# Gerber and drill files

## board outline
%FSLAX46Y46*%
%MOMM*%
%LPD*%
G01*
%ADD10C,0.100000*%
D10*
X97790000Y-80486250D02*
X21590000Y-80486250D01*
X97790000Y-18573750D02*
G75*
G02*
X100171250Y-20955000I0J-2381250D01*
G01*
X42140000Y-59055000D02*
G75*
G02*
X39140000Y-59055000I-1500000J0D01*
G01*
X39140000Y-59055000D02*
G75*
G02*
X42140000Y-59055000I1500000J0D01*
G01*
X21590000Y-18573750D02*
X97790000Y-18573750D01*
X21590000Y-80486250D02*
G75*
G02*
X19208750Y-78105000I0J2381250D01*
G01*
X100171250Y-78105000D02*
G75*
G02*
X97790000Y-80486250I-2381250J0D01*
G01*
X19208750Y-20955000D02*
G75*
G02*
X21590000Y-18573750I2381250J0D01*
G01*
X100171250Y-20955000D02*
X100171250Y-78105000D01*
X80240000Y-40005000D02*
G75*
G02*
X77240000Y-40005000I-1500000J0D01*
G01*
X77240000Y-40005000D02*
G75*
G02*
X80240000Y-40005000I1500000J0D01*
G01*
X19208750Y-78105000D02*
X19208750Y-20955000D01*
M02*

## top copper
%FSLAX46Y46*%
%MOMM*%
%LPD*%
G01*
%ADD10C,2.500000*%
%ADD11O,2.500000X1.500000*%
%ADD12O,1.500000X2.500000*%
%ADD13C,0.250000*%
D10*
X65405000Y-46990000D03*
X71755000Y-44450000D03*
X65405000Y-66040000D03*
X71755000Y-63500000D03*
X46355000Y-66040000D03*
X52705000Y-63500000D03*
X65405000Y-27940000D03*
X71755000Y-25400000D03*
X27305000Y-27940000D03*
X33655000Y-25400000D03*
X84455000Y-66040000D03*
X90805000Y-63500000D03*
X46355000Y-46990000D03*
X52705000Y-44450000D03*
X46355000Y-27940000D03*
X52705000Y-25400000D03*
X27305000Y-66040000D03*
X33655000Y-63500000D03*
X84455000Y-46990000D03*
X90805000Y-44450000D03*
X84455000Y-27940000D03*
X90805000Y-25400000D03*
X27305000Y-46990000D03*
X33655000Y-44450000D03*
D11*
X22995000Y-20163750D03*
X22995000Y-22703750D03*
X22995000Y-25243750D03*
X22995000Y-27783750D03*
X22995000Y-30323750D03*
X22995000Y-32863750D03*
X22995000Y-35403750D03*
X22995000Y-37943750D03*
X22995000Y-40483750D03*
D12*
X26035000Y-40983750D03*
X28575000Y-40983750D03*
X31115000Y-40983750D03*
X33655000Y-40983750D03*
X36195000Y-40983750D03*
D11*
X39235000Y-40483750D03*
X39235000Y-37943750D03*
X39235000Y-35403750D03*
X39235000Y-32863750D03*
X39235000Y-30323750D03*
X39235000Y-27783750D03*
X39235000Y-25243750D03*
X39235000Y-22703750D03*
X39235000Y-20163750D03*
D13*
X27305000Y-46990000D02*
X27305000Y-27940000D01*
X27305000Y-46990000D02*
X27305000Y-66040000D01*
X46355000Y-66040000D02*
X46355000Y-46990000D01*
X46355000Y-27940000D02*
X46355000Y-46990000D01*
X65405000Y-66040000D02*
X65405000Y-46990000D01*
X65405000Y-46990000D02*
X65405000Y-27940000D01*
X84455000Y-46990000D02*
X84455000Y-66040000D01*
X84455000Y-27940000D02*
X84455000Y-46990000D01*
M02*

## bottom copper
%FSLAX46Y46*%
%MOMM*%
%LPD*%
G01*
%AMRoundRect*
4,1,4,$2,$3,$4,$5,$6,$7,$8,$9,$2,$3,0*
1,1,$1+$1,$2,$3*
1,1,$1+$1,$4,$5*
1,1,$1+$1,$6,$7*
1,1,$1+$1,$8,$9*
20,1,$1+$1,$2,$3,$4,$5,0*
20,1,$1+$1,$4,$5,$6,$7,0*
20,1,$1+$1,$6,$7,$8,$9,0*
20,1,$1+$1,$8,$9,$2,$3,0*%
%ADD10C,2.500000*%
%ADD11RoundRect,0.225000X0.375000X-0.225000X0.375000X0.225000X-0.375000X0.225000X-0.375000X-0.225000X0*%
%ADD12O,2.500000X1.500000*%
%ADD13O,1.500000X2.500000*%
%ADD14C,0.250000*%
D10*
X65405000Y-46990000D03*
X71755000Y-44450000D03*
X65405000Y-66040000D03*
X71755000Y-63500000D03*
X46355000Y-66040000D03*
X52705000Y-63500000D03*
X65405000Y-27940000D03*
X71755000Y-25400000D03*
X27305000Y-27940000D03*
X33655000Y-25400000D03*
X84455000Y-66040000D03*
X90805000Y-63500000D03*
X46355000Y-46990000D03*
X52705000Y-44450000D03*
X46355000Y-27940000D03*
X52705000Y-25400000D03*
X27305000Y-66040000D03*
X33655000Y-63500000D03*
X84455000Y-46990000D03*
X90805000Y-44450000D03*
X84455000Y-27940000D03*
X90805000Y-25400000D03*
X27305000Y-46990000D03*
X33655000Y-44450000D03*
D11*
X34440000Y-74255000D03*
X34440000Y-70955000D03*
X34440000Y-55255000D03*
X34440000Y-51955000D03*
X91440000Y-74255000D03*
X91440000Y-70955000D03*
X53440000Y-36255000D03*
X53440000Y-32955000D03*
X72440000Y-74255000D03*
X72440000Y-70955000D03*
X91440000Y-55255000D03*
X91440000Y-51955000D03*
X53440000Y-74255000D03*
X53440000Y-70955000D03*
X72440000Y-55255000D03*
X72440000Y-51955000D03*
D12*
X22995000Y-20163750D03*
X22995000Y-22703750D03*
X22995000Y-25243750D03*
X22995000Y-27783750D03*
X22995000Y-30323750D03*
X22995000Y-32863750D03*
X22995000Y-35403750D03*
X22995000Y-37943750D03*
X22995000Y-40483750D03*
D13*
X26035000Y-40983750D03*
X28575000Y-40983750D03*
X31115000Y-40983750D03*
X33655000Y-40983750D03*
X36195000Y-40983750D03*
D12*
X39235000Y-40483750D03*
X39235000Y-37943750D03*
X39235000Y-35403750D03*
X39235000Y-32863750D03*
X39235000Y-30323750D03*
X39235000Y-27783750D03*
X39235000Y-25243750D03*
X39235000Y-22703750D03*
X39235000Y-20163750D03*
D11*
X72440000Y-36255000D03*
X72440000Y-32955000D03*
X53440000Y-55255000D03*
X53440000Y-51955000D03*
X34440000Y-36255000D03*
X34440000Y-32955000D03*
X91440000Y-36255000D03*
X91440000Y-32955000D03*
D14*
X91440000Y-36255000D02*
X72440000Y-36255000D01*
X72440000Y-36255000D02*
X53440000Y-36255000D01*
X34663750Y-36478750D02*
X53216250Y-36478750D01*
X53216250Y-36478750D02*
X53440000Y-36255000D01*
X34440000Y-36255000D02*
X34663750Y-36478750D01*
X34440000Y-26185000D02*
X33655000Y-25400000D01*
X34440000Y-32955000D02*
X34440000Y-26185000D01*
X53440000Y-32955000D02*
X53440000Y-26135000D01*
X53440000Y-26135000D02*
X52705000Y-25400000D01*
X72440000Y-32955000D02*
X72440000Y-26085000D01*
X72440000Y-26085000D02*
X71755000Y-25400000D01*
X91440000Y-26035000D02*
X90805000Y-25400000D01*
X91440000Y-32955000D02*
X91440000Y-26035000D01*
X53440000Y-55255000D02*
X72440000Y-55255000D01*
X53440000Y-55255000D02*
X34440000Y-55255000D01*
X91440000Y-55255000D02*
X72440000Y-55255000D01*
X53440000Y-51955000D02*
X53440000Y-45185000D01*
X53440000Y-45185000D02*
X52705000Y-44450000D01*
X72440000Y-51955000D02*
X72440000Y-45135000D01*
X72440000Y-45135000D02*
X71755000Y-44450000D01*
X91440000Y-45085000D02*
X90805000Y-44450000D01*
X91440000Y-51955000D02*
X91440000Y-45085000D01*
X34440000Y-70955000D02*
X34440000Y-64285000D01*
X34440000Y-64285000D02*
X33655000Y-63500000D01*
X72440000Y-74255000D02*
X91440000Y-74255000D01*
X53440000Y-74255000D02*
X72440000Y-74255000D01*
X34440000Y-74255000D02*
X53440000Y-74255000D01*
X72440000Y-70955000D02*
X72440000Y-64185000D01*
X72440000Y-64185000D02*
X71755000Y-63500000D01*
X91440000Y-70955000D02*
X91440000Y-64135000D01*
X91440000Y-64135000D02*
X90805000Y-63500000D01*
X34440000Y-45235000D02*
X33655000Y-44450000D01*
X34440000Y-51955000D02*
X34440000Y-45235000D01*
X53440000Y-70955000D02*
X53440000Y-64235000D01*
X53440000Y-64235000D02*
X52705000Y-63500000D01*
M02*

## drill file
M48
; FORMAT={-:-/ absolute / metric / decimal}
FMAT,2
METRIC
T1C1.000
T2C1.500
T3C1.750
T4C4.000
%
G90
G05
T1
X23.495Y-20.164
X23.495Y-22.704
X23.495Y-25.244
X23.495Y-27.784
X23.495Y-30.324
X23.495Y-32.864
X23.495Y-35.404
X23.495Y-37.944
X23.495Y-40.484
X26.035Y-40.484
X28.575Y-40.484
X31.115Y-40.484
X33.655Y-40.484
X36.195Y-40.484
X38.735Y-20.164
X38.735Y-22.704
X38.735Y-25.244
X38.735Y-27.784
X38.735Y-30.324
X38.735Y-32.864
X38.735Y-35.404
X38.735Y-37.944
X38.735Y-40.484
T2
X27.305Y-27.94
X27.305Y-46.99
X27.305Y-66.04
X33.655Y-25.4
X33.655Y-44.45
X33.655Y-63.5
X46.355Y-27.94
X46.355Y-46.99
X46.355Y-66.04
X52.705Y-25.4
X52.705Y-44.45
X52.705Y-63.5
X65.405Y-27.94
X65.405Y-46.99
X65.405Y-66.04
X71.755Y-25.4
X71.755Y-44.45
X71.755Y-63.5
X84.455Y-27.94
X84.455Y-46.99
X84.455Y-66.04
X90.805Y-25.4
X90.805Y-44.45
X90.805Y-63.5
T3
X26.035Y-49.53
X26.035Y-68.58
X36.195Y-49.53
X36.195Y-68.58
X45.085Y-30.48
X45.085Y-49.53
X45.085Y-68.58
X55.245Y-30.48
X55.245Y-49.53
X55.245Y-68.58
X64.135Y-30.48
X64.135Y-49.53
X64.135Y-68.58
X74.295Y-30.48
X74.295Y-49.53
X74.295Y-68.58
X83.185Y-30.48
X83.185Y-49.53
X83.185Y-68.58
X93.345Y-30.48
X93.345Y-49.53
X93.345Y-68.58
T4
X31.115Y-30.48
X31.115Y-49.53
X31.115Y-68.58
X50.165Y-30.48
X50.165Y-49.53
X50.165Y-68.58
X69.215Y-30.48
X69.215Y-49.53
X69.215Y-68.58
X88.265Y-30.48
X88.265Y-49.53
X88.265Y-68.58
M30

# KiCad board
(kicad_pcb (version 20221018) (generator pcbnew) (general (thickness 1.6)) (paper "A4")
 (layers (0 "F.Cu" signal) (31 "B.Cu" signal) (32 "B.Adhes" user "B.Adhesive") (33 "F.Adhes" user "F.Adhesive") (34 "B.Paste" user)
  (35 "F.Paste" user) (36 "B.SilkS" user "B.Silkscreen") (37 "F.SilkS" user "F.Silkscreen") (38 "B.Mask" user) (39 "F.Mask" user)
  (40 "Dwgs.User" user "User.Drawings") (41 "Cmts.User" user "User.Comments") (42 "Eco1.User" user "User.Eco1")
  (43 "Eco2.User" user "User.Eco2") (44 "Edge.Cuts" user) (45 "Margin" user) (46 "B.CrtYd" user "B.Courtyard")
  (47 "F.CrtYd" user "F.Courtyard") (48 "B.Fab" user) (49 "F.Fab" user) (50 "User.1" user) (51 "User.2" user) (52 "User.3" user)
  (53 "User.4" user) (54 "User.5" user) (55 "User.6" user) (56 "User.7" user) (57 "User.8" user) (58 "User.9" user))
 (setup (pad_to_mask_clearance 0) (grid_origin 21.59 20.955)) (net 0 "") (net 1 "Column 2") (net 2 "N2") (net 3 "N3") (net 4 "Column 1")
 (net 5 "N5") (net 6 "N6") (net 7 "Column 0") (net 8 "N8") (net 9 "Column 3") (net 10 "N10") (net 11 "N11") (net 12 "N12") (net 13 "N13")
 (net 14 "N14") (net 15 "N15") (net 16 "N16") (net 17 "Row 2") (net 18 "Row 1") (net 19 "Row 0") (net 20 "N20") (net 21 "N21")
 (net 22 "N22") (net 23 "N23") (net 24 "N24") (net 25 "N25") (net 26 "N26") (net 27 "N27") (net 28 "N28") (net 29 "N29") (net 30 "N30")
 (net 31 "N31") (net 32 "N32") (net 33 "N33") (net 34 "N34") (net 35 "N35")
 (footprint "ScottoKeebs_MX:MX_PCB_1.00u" (layer "F.Cu") (at 69.215 49.53)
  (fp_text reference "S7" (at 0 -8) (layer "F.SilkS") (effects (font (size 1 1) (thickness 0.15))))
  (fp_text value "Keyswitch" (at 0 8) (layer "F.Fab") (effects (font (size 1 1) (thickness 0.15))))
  (pad "" np_thru_hole circle (at -5.08 0) (size 1.75 1.75) (drill 1.75) (layers "*.Cu" "*.Mask"))
  (pad "" np_thru_hole circle (at 0 0) (size 4 4) (drill 4) (layers "*.Cu" "*.Mask"))
  (pad "" np_thru_hole circle (at 5.08 0) (size 1.75 1.75) (drill 1.75) (layers "*.Cu" "*.Mask"))
  (pad "1" thru_hole circle (at -3.81 -2.54) (size 2.5 2.5) (drill 1.5) (layers "*.Cu" "*.Mask") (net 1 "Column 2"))
  (pad "2" thru_hole circle (at 2.54 -5.08) (size 2.5 2.5) (drill 1.5) (layers "*.Cu" "*.Mask") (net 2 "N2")))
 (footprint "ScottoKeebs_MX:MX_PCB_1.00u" (layer "F.Cu") (at 69.215 68.58)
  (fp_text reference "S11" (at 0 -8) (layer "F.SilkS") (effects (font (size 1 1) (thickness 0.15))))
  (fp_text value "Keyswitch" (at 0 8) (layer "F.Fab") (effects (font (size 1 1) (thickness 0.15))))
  (pad "" np_thru_hole circle (at -5.08 0) (size 1.75 1.75) (drill 1.75) (layers "*.Cu" "*.Mask"))
  (pad "" np_thru_hole circle (at 0 0) (size 4 4) (drill 4) (layers "*.Cu" "*.Mask"))
  (pad "" np_thru_hole circle (at 5.08 0) (size 1.75 1.75) (drill 1.75) (layers "*.Cu" "*.Mask"))
  (pad "1" thru_hole circle (at -3.81 -2.54) (size 2.5 2.5) (drill 1.5) (layers "*.Cu" "*.Mask") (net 1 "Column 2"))
  (pad "2" thru_hole circle (at 2.54 -5.08) (size 2.5 2.5) (drill 1.5) (layers "*.Cu" "*.Mask") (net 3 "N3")))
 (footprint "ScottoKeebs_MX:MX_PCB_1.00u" (layer "F.Cu") (at 50.165 68.58)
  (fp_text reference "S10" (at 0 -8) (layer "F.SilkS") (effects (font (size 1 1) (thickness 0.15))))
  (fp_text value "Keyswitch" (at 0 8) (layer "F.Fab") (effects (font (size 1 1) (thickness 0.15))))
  (pad "" np_thru_hole circle (at -5.08 0) (size 1.75 1.75) (drill 1.75) (layers "*.Cu" "*.Mask"))
  (pad "" np_thru_hole circle (at 0 0) (size 4 4) (drill 4) (layers "*.Cu" "*.Mask"))
  (pad "" np_thru_hole circle (at 5.08 0) (size 1.75 1.75) (drill 1.75) (layers "*.Cu" "*.Mask"))
  (pad "1" thru_hole circle (at -3.81 -2.54) (size 2.5 2.5) (drill 1.5) (layers "*.Cu" "*.Mask") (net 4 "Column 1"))
  (pad "2" thru_hole circle (at 2.54 -5.08) (size 2.5 2.5) (drill 1.5) (layers "*.Cu" "*.Mask") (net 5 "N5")))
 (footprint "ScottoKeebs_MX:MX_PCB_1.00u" (layer "F.Cu") (at 69.215 30.48)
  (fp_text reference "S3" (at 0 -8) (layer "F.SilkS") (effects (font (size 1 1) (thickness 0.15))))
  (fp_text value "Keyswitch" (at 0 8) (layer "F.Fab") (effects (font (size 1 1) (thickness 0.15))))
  (pad "" np_thru_hole circle (at -5.08 0) (size 1.75 1.75) (drill 1.75) (layers "*.Cu" "*.Mask"))
  (pad "" np_thru_hole circle (at 0 0) (size 4 4) (drill 4) (layers "*.Cu" "*.Mask"))
  (pad "" np_thru_hole circle (at 5.08 0) (size 1.75 1.75) (drill 1.75) (layers "*.Cu" "*.Mask"))
  (pad "1" thru_hole circle (at -3.81 -2.54) (size 2.5 2.5) (drill 1.5) (layers "*.Cu" "*.Mask") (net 1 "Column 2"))
  (pad "2" thru_hole circle (at 2.54 -5.08) (size 2.5 2.5) (drill 1.5) (layers "*.Cu" "*.Mask") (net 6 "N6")))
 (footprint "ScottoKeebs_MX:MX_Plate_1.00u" (layer "F.Cu") (at 31.115 30.48)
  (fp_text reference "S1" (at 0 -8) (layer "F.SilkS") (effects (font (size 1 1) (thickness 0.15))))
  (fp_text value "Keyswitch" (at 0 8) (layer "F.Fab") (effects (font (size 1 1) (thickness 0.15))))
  (pad "" np_thru_hole circle (at 0 0) (size 4 4) (drill 4) (layers "*.Cu" "*.Mask"))
  (pad "1" thru_hole circle (at -3.81 -2.54) (size 2.5 2.5) (drill 1.5) (layers "*.Cu" "*.Mask") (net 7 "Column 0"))
  (pad "2" thru_hole circle (at 2.54 -5.08) (size 2.5 2.5) (drill 1.5) (layers "*.Cu" "*.Mask") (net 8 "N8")))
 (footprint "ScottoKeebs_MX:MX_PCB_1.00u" (layer "F.Cu") (at 88.265 68.58)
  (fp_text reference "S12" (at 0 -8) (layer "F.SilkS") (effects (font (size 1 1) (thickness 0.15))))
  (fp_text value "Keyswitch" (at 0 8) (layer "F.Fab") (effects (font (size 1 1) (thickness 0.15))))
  (pad "" np_thru_hole circle (at -5.08 0) (size 1.75 1.75) (drill 1.75) (layers "*.Cu" "*.Mask"))
  (pad "" np_thru_hole circle (at 0 0) (size 4 4) (drill 4) (layers "*.Cu" "*.Mask"))
  (pad "" np_thru_hole circle (at 5.08 0) (size 1.75 1.75) (drill 1.75) (layers "*.Cu" "*.Mask"))
  (pad "1" thru_hole circle (at -3.81 -2.54) (size 2.5 2.5) (drill 1.5) (layers "*.Cu" "*.Mask") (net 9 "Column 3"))
  (pad "2" thru_hole circle (at 2.54 -5.08) (size 2.5 2.5) (drill 1.5) (layers "*.Cu" "*.Mask") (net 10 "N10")))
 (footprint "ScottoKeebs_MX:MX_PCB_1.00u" (layer "F.Cu") (at 50.165 49.53)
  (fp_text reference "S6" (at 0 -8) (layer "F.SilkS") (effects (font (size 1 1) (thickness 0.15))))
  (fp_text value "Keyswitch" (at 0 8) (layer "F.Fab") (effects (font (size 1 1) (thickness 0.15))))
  (pad "" np_thru_hole circle (at -5.08 0) (size 1.75 1.75) (drill 1.75) (layers "*.Cu" "*.Mask"))
  (pad "" np_thru_hole circle (at 0 0) (size 4 4) (drill 4) (layers "*.Cu" "*.Mask"))
  (pad "" np_thru_hole circle (at 5.08 0) (size 1.75 1.75) (drill 1.75) (layers "*.Cu" "*.Mask"))
  (pad "1" thru_hole circle (at -3.81 -2.54) (size 2.5 2.5) (drill 1.5) (layers "*.Cu" "*.Mask") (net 4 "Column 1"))
  (pad "2" thru_hole circle (at 2.54 -5.08) (size 2.5 2.5) (drill 1.5) (layers "*.Cu" "*.Mask") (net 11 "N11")))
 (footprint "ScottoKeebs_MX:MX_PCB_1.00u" (layer "F.Cu") (at 50.165 30.48)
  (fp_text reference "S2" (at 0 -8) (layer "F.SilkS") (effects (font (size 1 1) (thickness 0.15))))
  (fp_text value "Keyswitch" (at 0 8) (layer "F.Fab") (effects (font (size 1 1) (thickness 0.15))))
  (pad "" np_thru_hole circle (at -5.08 0) (size 1.75 1.75) (drill 1.75) (layers "*.Cu" "*.Mask"))
  (pad "" np_thru_hole circle (at 0 0) (size 4 4) (drill 4) (layers "*.Cu" "*.Mask"))
  (pad "" np_thru_hole circle (at 5.08 0) (size 1.75 1.75) (drill 1.75) (layers "*.Cu" "*.Mask"))
  (pad "1" thru_hole circle (at -3.81 -2.54) (size 2.5 2.5) (drill 1.5) (layers "*.Cu" "*.Mask") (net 4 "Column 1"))
  (pad "2" thru_hole circle (at 2.54 -5.08) (size 2.5 2.5) (drill 1.5) (layers "*.Cu" "*.Mask") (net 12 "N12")))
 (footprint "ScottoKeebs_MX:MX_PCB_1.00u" (layer "F.Cu") (at 31.115 68.58)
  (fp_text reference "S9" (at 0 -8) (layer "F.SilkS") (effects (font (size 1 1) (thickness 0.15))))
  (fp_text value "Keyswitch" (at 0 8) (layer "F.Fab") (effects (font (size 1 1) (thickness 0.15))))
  (pad "" np_thru_hole circle (at -5.08 0) (size 1.75 1.75) (drill 1.75) (layers "*.Cu" "*.Mask"))
  (pad "" np_thru_hole circle (at 0 0) (size 4 4) (drill 4) (layers "*.Cu" "*.Mask"))
  (pad "" np_thru_hole circle (at 5.08 0) (size 1.75 1.75) (drill 1.75) (layers "*.Cu" "*.Mask"))
  (pad "1" thru_hole circle (at -3.81 -2.54) (size 2.5 2.5) (drill 1.5) (layers "*.Cu" "*.Mask") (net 7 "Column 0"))
  (pad "2" thru_hole circle (at 2.54 -5.08) (size 2.5 2.5) (drill 1.5) (layers "*.Cu" "*.Mask") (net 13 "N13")))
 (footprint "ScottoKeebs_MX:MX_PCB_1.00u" (layer "F.Cu") (at 88.265 49.53)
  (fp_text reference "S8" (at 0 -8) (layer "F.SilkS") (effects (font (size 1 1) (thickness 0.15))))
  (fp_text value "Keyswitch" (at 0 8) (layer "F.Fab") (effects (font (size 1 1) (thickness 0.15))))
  (pad "" np_thru_hole circle (at -5.08 0) (size 1.75 1.75) (drill 1.75) (layers "*.Cu" "*.Mask"))
  (pad "" np_thru_hole circle (at 0 0) (size 4 4) (drill 4) (layers "*.Cu" "*.Mask"))
  (pad "" np_thru_hole circle (at 5.08 0) (size 1.75 1.75) (drill 1.75) (layers "*.Cu" "*.Mask"))
  (pad "1" thru_hole circle (at -3.81 -2.54) (size 2.5 2.5) (drill 1.5) (layers "*.Cu" "*.Mask") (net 9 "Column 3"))
  (pad "2" thru_hole circle (at 2.54 -5.08) (size 2.5 2.5) (drill 1.5) (layers "*.Cu" "*.Mask") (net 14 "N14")))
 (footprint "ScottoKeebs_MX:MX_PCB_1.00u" (layer "F.Cu") (at 88.265 30.48)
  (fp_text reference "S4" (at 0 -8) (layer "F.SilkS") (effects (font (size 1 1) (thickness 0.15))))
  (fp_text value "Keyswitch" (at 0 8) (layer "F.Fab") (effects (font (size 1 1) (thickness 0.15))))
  (pad "" np_thru_hole circle (at -5.08 0) (size 1.75 1.75) (drill 1.75) (layers "*.Cu" "*.Mask"))
  (pad "" np_thru_hole circle (at 0 0) (size 4 4) (drill 4) (layers "*.Cu" "*.Mask"))
  (pad "" np_thru_hole circle (at 5.08 0) (size 1.75 1.75) (drill 1.75) (layers "*.Cu" "*.Mask"))
  (pad "1" thru_hole circle (at -3.81 -2.54) (size 2.5 2.5) (drill 1.5) (layers "*.Cu" "*.Mask") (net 9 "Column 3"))
  (pad "2" thru_hole circle (at 2.54 -5.08) (size 2.5 2.5) (drill 1.5) (layers "*.Cu" "*.Mask") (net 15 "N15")))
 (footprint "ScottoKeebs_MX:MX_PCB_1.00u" (layer "F.Cu") (at 31.115 49.53)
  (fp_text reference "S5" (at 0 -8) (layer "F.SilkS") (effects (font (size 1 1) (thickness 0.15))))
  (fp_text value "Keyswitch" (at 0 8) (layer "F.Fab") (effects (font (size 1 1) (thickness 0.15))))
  (pad "" np_thru_hole circle (at -5.08 0) (size 1.75 1.75) (drill 1.75) (layers "*.Cu" "*.Mask"))
  (pad "" np_thru_hole circle (at 0 0) (size 4 4) (drill 4) (layers "*.Cu" "*.Mask"))
  (pad "" np_thru_hole circle (at 5.08 0) (size 1.75 1.75) (drill 1.75) (layers "*.Cu" "*.Mask"))
  (pad "1" thru_hole circle (at -3.81 -2.54) (size 2.5 2.5) (drill 1.5) (layers "*.Cu" "*.Mask") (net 7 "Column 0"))
  (pad "2" thru_hole circle (at 2.54 -5.08) (size 2.5 2.5) (drill 1.5) (layers "*.Cu" "*.Mask") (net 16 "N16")))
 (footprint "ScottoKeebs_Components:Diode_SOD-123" (layer "B.Cu") (at 34.44 72.605 90)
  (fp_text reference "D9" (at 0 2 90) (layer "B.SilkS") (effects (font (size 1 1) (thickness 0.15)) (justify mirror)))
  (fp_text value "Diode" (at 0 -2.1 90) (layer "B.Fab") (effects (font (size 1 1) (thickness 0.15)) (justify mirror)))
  (pad "1" smd roundrect (at -1.65 0 90) (size 0.9 1.2) (layers "B.Cu" "B.Paste" "B.Mask") (roundrect_rratio 0.25) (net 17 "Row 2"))
  (pad "2" smd roundrect (at 1.65 0 90) (size 0.9 1.2) (layers "B.Cu" "B.Paste" "B.Mask") (roundrect_rratio 0.25) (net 13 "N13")))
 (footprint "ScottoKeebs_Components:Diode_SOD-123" (layer "B.Cu") (at 34.44 53.605 90)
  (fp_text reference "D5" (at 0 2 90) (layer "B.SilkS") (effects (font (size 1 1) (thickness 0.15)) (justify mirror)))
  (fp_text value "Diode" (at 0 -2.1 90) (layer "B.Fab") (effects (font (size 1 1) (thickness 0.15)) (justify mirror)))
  (pad "1" smd roundrect (at -1.65 0 90) (size 0.9 1.2) (layers "B.Cu" "B.Paste" "B.Mask") (roundrect_rratio 0.25) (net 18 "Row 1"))
  (pad "2" smd roundrect (at 1.65 0 90) (size 0.9 1.2) (layers "B.Cu" "B.Paste" "B.Mask") (roundrect_rratio 0.25) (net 16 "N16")))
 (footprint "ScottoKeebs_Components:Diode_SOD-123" (layer "B.Cu") (at 91.44 72.605 90)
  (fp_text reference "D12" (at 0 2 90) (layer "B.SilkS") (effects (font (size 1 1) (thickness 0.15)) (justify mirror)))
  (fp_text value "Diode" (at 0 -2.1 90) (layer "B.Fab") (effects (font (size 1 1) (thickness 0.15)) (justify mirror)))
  (pad "1" smd roundrect (at -1.65 0 90) (size 0.9 1.2) (layers "B.Cu" "B.Paste" "B.Mask") (roundrect_rratio 0.25) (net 17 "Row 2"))
  (pad "2" smd roundrect (at 1.65 0 90) (size 0.9 1.2) (layers "B.Cu" "B.Paste" "B.Mask") (roundrect_rratio 0.25) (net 10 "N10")))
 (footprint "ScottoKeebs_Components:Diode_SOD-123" (layer "B.Cu") (at 53.44 34.605 90)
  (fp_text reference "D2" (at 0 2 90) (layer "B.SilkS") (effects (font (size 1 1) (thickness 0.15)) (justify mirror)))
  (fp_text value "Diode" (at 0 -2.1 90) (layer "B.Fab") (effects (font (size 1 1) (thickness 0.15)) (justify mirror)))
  (pad "1" smd roundrect (at -1.65 0 90) (size 0.9 1.2) (layers "B.Cu" "B.Paste" "B.Mask") (roundrect_rratio 0.25) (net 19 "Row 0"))
  (pad "2" smd roundrect (at 1.65 0 90) (size 0.9 1.2) (layers "B.Cu" "B.Paste" "B.Mask") (roundrect_rratio 0.25) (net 12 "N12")))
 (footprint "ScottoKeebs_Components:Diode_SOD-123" (layer "B.Cu") (at 72.44 72.605 90)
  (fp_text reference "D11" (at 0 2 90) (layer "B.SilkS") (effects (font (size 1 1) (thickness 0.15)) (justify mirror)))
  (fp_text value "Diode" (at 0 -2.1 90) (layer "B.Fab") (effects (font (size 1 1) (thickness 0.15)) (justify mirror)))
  (pad "1" smd roundrect (at -1.65 0 90) (size 0.9 1.2) (layers "B.Cu" "B.Paste" "B.Mask") (roundrect_rratio 0.25) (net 17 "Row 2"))
  (pad "2" smd roundrect (at 1.65 0 90) (size 0.9 1.2) (layers "B.Cu" "B.Paste" "B.Mask") (roundrect_rratio 0.25) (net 3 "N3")))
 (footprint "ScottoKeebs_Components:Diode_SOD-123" (layer "B.Cu") (at 91.44 53.605 90)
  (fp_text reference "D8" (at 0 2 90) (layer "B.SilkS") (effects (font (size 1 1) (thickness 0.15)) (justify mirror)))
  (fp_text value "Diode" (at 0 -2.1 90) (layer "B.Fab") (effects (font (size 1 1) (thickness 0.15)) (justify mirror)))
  (pad "1" smd roundrect (at -1.65 0 90) (size 0.9 1.2) (layers "B.Cu" "B.Paste" "B.Mask") (roundrect_rratio 0.25) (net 18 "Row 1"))
  (pad "2" smd roundrect (at 1.65 0 90) (size 0.9 1.2) (layers "B.Cu" "B.Paste" "B.Mask") (roundrect_rratio 0.25) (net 14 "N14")))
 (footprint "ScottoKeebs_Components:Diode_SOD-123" (layer "B.Cu") (at 53.44 72.605 90)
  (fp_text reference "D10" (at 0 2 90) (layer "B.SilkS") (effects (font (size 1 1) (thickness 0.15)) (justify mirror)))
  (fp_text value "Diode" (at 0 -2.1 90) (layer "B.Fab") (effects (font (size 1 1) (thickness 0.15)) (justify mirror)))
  (pad "1" smd roundrect (at -1.65 0 90) (size 0.9 1.2) (layers "B.Cu" "B.Paste" "B.Mask") (roundrect_rratio 0.25) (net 17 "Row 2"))
  (pad "2" smd roundrect (at 1.65 0 90) (size 0.9 1.2) (layers "B.Cu" "B.Paste" "B.Mask") (roundrect_rratio 0.25) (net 5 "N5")))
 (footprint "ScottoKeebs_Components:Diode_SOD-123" (layer "B.Cu") (at 72.44 53.605 90)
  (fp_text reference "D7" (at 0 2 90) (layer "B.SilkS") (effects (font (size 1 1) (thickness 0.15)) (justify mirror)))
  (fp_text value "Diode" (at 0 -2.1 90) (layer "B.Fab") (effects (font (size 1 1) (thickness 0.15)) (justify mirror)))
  (pad "1" smd roundrect (at -1.65 0 90) (size 0.9 1.2) (layers "B.Cu" "B.Paste" "B.Mask") (roundrect_rratio 0.25) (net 18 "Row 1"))
  (pad "2" smd roundrect (at 1.65 0 90) (size 0.9 1.2) (layers "B.Cu" "B.Paste" "B.Mask") (roundrect_rratio 0.25) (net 2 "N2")))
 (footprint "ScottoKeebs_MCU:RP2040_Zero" (layer "B.Cu") (at 31.115 30.32375 180)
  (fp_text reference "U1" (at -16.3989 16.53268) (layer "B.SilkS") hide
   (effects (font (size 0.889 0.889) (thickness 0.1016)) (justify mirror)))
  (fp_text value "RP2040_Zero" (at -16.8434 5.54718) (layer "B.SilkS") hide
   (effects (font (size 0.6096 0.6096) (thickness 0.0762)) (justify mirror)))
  (pad "1" thru_hole oval (at 7.62 10.16) (size 2.5 1.5) (drill 1 (offset -0.5 0)) (layers "*.Cu" "*.Mask") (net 7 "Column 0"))
  (pad "2" thru_hole oval (at 7.62 7.62) (size 2.5 1.5) (drill 1 (offset -0.5 0)) (layers "*.Cu" "*.Mask") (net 4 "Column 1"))
  (pad "3" thru_hole oval (at 7.62 5.08) (size 2.5 1.5) (drill 1 (offset -0.5 0)) (layers "*.Cu" "*.Mask") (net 1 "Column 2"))
  (pad "4" thru_hole oval (at 7.62 2.54) (size 2.5 1.5) (drill 1 (offset -0.5 0)) (layers "*.Cu" "*.Mask") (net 9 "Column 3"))
  (pad "5" thru_hole oval (at 7.62 0) (size 2.5 1.5) (drill 1 (offset -0.5 0)) (layers "*.Cu" "*.Mask") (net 19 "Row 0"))
  (pad "6" thru_hole oval (at 7.62 -2.54) (size 2.5 1.5) (drill 1 (offset -0.5 0)) (layers "*.Cu" "*.Mask") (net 18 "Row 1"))
  (pad "7" thru_hole oval (at 7.62 -5.08) (size 2.5 1.5) (drill 1 (offset -0.5 0)) (layers "*.Cu" "*.Mask") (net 17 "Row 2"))
  (pad "8" thru_hole oval (at 7.62 -7.62) (size 2.5 1.5) (drill 1 (offset -0.5 0)) (layers "*.Cu" "*.Mask") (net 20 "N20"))
  (pad "9" thru_hole oval (at 7.62 -10.16) (size 2.5 1.5) (drill 1 (offset -0.5 0)) (layers "*.Cu" "*.Mask") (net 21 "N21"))
  (pad "10" thru_hole oval (at 5.08 -10.16 90) (size 2.5 1.5) (drill 1 (offset -0.5 0)) (layers "*.Cu" "*.Mask") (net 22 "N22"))
  (pad "11" thru_hole oval (at 2.54 -10.16 90) (size 2.5 1.5) (drill 1 (offset -0.5 0)) (layers "*.Cu" "*.Mask") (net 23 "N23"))
  (pad "12" thru_hole oval (at 0 -10.16 90) (size 2.5 1.5) (drill 1 (offset -0.5 0)) (layers "*.Cu" "*.Mask") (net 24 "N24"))
  (pad "13" thru_hole oval (at -2.54 -10.16 90) (size 2.5 1.5) (drill 1 (offset -0.5 0)) (layers "*.Cu" "*.Mask") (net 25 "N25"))
  (pad "14" thru_hole oval (at -5.08 -10.16 90) (size 2.5 1.5) (drill 1 (offset -0.5 0)) (layers "*.Cu" "*.Mask") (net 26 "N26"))
  (pad "15" thru_hole oval (at -7.62 -10.16 180) (size 2.5 1.5) (drill 1 (offset -0.5 0)) (layers "*.Cu" "*.Mask") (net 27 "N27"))
  (pad "16" thru_hole oval (at -7.62 -7.62 180) (size 2.5 1.5) (drill 1 (offset -0.5 0)) (layers "*.Cu" "*.Mask") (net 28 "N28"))
  (pad "17" thru_hole oval (at -7.62 -5.08 180) (size 2.5 1.5) (drill 1 (offset -0.5 0)) (layers "*.Cu" "*.Mask") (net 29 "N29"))
  (pad "18" thru_hole oval (at -7.62 -2.54 180) (size 2.5 1.5) (drill 1 (offset -0.5 0)) (layers "*.Cu" "*.Mask") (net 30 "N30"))
  (pad "19" thru_hole oval (at -7.62 0 180) (size 2.5 1.5) (drill 1 (offset -0.5 0)) (layers "*.Cu" "*.Mask") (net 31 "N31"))
  (pad "20" thru_hole oval (at -7.62 2.54 180) (size 2.5 1.5) (drill 1 (offset -0.5 0)) (layers "*.Cu" "*.Mask") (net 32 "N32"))
  (pad "21" thru_hole oval (at -7.62 5.08 180) (size 2.5 1.5) (drill 1 (offset -0.5 0)) (layers "*.Cu" "*.Mask") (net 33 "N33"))
  (pad "22" thru_hole oval (at -7.62 7.62 180) (size 2.5 1.5) (drill 1 (offset -0.5 0)) (layers "*.Cu" "*.Mask") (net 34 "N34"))
  (pad "23" thru_hole oval (at -7.62 10.16 180) (size 2.5 1.5) (drill 1 (offset -0.5 0)) (layers "*.Cu" "*.Mask") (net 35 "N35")))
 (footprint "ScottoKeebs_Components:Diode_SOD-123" (layer "B.Cu") (at 72.44 34.605 90)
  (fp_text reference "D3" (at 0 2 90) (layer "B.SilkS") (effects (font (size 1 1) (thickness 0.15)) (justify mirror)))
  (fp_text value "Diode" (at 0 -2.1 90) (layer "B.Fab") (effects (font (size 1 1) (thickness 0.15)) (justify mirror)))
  (pad "1" smd roundrect (at -1.65 0 90) (size 0.9 1.2) (layers "B.Cu" "B.Paste" "B.Mask") (roundrect_rratio 0.25) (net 19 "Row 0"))
  (pad "2" smd roundrect (at 1.65 0 90) (size 0.9 1.2) (layers "B.Cu" "B.Paste" "B.Mask") (roundrect_rratio 0.25) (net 6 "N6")))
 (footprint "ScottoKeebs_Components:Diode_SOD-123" (layer "B.Cu") (at 53.44 53.605 90)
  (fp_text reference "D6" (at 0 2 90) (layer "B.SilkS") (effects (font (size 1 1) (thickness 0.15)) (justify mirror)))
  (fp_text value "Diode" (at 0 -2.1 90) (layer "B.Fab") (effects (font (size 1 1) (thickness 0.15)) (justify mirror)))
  (pad "1" smd roundrect (at -1.65 0 90) (size 0.9 1.2) (layers "B.Cu" "B.Paste" "B.Mask") (roundrect_rratio 0.25) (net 18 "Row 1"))
  (pad "2" smd roundrect (at 1.65 0 90) (size 0.9 1.2) (layers "B.Cu" "B.Paste" "B.Mask") (roundrect_rratio 0.25) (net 11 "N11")))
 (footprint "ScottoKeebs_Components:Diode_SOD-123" (layer "B.Cu") (at 34.44 34.605 90)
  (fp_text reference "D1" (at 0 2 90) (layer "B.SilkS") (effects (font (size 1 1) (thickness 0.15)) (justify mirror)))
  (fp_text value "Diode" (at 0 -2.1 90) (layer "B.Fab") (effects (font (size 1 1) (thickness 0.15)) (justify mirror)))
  (pad "1" smd roundrect (at -1.65 0 90) (size 0.9 1.2) (layers "B.Cu" "B.Paste" "B.Mask") (roundrect_rratio 0.25) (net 19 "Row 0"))
  (pad "2" smd roundrect (at 1.65 0 90) (size 0.9 1.2) (layers "B.Cu" "B.Paste" "B.Mask") (roundrect_rratio 0.25) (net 8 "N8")))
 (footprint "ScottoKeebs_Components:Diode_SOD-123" (layer "B.Cu") (at 91.44 34.605 90)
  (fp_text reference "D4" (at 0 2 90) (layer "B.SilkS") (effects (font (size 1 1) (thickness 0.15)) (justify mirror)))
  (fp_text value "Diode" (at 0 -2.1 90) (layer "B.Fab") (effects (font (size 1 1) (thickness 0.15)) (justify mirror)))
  (pad "1" smd roundrect (at -1.65 0 90) (size 0.9 1.2) (layers "B.Cu" "B.Paste" "B.Mask") (roundrect_rratio 0.25) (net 19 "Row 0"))
  (pad "2" smd roundrect (at 1.65 0 90) (size 0.9 1.2) (layers "B.Cu" "B.Paste" "B.Mask") (roundrect_rratio 0.25) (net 15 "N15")))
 (gr_line (start 97.79 80.48625) (end 21.59 80.48625) (stroke (width 0.1) (type default)) (layer "Edge.Cuts"))
 (gr_arc (start 97.79 18.57375) (mid 99.473798 19.271202) (end 100.17125 20.955) (stroke (width 0.1) (type default)) (layer "Edge.Cuts"))
 (gr_circle (center 40.64 59.055) (end 42.14 59.055) (stroke (width 0.1) (type default)) (fill none) (layer "Edge.Cuts"))
 (gr_line (start 21.59 18.57375) (end 97.79 18.57375) (stroke (width 0.1) (type default)) (layer "Edge.Cuts"))
 (gr_arc (start 21.59 80.48625) (mid 19.906202 79.788798) (end 19.20875 78.105) (stroke (width 0.1) (type default)) (layer "Edge.Cuts"))
 (gr_arc (start 100.17125 78.105) (mid 99.473798 79.788798) (end 97.79 80.48625) (stroke (width 0.1) (type default)) (layer "Edge.Cuts"))
 (gr_arc (start 19.20875 20.955) (mid 19.906202 19.271202) (end 21.59 18.57375) (stroke (width 0.1) (type default)) (layer "Edge.Cuts"))
 (gr_line (start 100.17125 20.955) (end 100.17125 78.105) (stroke (width 0.1) (type default)) (layer "Edge.Cuts"))
 (gr_circle (center 78.74 40.005) (end 80.24 40.005) (stroke (width 0.1) (type default)) (fill none) (layer "Edge.Cuts"))
 (gr_line (start 19.20875 78.105) (end 19.20875 20.955) (stroke (width 0.1) (type default)) (layer "Edge.Cuts"))
 (segment (start 91.44 36.255) (end 72.44 36.255) (width 0.25) (layer "B.Cu") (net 19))
 (segment (start 72.44 36.255) (end 53.44 36.255) (width 0.25) (layer "B.Cu") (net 19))
 (segment (start 34.66375 36.47875) (end 53.21625 36.47875) (width 0.25) (layer "B.Cu") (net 19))
 (segment (start 53.21625 36.47875) (end 53.44 36.255) (width 0.25) (layer "B.Cu") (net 19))
 (segment (start 34.44 36.255) (end 34.66375 36.47875) (width 0.25) (layer "B.Cu") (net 19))
 (segment (start 34.44 26.185) (end 33.655 25.4) (width 0.25) (layer "B.Cu") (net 8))
 (segment (start 34.44 32.955) (end 34.44 26.185) (width 0.25) (layer "B.Cu") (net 8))
 (segment (start 53.44 32.955) (end 53.44 26.135) (width 0.25) (layer "B.Cu") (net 12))
 (segment (start 53.44 26.135) (end 52.705 25.4) (width 0.25) (layer "B.Cu") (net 12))
 (segment (start 72.44 32.955) (end 72.44 26.085) (width 0.25) (layer "B.Cu") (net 6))
 (segment (start 72.44 26.085) (end 71.755 25.4) (width 0.25) (layer "B.Cu") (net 6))
 (segment (start 91.44 26.035) (end 90.805 25.4) (width 0.25) (layer "B.Cu") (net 15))
 (segment (start 91.44 32.955) (end 91.44 26.035) (width 0.25) (layer "B.Cu") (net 15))
 (segment (start 53.44 55.255) (end 72.44 55.255) (width 0.25) (layer "B.Cu") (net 18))
 (segment (start 53.44 55.255) (end 34.44 55.255) (width 0.25) (layer "B.Cu") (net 18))
 (segment (start 91.44 55.255) (end 72.44 55.255) (width 0.25) (layer "B.Cu") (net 18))
 (segment (start 53.44 51.955) (end 53.44 45.185) (width 0.25) (layer "B.Cu") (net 11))
 (segment (start 53.44 45.185) (end 52.705 44.45) (width 0.25) (layer "B.Cu") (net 11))
 (segment (start 72.44 51.955) (end 72.44 45.135) (width 0.25) (layer "B.Cu") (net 2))
 (segment (start 72.44 45.135) (end 71.755 44.45) (width 0.25) (layer "B.Cu") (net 2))
 (segment (start 91.44 45.085) (end 90.805 44.45) (width 0.25) (layer "B.Cu") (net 14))
 (segment (start 91.44 51.955) (end 91.44 45.085) (width 0.25) (layer "B.Cu") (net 14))
 (segment (start 34.44 70.955) (end 34.44 64.285) (width 0.25) (layer "B.Cu") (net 13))
 (segment (start 34.44 64.285) (end 33.655 63.5) (width 0.25) (layer "B.Cu") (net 13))
 (segment (start 72.44 74.255) (end 91.44 74.255) (width 0.25) (layer "B.Cu") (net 17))
 (segment (start 53.44 74.255) (end 72.44 74.255) (width 0.25) (layer "B.Cu") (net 17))
 (segment (start 34.44 74.255) (end 53.44 74.255) (width 0.25) (layer "B.Cu") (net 17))
 (segment (start 72.44 70.955) (end 72.44 64.185) (width 0.25) (layer "B.Cu") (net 3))
 (segment (start 72.44 64.185) (end 71.755 63.5) (width 0.25) (layer "B.Cu") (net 3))
 (segment (start 91.44 70.955) (end 91.44 64.135) (width 0.25) (layer "B.Cu") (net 10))
 (segment (start 91.44 64.135) (end 90.805 63.5) (width 0.25) (layer "B.Cu") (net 10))
 (segment (start 27.305 46.99) (end 27.305 27.94) (width 0.25) (layer "F.Cu") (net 7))
 (segment (start 27.305 46.99) (end 27.305 66.04) (width 0.25) (layer "F.Cu") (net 7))
 (segment (start 46.355 66.04) (end 46.355 46.99) (width 0.25) (layer "F.Cu") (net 4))
 (segment (start 46.355 27.94) (end 46.355 46.99) (width 0.25) (layer "F.Cu") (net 4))
 (segment (start 65.405 66.04) (end 65.405 46.99) (width 0.25) (layer "F.Cu") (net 1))
 (segment (start 65.405 46.99) (end 65.405 27.94) (width 0.25) (layer "F.Cu") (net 1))
 (segment (start 84.455 46.99) (end 84.455 66.04) (width 0.25) (layer "F.Cu") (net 9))
 (segment (start 84.455 27.94) (end 84.455 46.99) (width 0.25) (layer "F.Cu") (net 9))
 (segment (start 34.44 45.235) (end 33.655 44.45) (width 0.25) (layer "B.Cu") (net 16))
 (segment (start 34.44 51.955) (end 34.44 45.235) (width 0.25) (layer "B.Cu") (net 16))
 (segment (start 53.44 70.955) (end 53.44 64.235) (width 0.25) (layer "B.Cu") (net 5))
 (segment (start 53.44 64.235) (end 52.705 63.5) (width 0.25) (layer "B.Cu") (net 5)))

